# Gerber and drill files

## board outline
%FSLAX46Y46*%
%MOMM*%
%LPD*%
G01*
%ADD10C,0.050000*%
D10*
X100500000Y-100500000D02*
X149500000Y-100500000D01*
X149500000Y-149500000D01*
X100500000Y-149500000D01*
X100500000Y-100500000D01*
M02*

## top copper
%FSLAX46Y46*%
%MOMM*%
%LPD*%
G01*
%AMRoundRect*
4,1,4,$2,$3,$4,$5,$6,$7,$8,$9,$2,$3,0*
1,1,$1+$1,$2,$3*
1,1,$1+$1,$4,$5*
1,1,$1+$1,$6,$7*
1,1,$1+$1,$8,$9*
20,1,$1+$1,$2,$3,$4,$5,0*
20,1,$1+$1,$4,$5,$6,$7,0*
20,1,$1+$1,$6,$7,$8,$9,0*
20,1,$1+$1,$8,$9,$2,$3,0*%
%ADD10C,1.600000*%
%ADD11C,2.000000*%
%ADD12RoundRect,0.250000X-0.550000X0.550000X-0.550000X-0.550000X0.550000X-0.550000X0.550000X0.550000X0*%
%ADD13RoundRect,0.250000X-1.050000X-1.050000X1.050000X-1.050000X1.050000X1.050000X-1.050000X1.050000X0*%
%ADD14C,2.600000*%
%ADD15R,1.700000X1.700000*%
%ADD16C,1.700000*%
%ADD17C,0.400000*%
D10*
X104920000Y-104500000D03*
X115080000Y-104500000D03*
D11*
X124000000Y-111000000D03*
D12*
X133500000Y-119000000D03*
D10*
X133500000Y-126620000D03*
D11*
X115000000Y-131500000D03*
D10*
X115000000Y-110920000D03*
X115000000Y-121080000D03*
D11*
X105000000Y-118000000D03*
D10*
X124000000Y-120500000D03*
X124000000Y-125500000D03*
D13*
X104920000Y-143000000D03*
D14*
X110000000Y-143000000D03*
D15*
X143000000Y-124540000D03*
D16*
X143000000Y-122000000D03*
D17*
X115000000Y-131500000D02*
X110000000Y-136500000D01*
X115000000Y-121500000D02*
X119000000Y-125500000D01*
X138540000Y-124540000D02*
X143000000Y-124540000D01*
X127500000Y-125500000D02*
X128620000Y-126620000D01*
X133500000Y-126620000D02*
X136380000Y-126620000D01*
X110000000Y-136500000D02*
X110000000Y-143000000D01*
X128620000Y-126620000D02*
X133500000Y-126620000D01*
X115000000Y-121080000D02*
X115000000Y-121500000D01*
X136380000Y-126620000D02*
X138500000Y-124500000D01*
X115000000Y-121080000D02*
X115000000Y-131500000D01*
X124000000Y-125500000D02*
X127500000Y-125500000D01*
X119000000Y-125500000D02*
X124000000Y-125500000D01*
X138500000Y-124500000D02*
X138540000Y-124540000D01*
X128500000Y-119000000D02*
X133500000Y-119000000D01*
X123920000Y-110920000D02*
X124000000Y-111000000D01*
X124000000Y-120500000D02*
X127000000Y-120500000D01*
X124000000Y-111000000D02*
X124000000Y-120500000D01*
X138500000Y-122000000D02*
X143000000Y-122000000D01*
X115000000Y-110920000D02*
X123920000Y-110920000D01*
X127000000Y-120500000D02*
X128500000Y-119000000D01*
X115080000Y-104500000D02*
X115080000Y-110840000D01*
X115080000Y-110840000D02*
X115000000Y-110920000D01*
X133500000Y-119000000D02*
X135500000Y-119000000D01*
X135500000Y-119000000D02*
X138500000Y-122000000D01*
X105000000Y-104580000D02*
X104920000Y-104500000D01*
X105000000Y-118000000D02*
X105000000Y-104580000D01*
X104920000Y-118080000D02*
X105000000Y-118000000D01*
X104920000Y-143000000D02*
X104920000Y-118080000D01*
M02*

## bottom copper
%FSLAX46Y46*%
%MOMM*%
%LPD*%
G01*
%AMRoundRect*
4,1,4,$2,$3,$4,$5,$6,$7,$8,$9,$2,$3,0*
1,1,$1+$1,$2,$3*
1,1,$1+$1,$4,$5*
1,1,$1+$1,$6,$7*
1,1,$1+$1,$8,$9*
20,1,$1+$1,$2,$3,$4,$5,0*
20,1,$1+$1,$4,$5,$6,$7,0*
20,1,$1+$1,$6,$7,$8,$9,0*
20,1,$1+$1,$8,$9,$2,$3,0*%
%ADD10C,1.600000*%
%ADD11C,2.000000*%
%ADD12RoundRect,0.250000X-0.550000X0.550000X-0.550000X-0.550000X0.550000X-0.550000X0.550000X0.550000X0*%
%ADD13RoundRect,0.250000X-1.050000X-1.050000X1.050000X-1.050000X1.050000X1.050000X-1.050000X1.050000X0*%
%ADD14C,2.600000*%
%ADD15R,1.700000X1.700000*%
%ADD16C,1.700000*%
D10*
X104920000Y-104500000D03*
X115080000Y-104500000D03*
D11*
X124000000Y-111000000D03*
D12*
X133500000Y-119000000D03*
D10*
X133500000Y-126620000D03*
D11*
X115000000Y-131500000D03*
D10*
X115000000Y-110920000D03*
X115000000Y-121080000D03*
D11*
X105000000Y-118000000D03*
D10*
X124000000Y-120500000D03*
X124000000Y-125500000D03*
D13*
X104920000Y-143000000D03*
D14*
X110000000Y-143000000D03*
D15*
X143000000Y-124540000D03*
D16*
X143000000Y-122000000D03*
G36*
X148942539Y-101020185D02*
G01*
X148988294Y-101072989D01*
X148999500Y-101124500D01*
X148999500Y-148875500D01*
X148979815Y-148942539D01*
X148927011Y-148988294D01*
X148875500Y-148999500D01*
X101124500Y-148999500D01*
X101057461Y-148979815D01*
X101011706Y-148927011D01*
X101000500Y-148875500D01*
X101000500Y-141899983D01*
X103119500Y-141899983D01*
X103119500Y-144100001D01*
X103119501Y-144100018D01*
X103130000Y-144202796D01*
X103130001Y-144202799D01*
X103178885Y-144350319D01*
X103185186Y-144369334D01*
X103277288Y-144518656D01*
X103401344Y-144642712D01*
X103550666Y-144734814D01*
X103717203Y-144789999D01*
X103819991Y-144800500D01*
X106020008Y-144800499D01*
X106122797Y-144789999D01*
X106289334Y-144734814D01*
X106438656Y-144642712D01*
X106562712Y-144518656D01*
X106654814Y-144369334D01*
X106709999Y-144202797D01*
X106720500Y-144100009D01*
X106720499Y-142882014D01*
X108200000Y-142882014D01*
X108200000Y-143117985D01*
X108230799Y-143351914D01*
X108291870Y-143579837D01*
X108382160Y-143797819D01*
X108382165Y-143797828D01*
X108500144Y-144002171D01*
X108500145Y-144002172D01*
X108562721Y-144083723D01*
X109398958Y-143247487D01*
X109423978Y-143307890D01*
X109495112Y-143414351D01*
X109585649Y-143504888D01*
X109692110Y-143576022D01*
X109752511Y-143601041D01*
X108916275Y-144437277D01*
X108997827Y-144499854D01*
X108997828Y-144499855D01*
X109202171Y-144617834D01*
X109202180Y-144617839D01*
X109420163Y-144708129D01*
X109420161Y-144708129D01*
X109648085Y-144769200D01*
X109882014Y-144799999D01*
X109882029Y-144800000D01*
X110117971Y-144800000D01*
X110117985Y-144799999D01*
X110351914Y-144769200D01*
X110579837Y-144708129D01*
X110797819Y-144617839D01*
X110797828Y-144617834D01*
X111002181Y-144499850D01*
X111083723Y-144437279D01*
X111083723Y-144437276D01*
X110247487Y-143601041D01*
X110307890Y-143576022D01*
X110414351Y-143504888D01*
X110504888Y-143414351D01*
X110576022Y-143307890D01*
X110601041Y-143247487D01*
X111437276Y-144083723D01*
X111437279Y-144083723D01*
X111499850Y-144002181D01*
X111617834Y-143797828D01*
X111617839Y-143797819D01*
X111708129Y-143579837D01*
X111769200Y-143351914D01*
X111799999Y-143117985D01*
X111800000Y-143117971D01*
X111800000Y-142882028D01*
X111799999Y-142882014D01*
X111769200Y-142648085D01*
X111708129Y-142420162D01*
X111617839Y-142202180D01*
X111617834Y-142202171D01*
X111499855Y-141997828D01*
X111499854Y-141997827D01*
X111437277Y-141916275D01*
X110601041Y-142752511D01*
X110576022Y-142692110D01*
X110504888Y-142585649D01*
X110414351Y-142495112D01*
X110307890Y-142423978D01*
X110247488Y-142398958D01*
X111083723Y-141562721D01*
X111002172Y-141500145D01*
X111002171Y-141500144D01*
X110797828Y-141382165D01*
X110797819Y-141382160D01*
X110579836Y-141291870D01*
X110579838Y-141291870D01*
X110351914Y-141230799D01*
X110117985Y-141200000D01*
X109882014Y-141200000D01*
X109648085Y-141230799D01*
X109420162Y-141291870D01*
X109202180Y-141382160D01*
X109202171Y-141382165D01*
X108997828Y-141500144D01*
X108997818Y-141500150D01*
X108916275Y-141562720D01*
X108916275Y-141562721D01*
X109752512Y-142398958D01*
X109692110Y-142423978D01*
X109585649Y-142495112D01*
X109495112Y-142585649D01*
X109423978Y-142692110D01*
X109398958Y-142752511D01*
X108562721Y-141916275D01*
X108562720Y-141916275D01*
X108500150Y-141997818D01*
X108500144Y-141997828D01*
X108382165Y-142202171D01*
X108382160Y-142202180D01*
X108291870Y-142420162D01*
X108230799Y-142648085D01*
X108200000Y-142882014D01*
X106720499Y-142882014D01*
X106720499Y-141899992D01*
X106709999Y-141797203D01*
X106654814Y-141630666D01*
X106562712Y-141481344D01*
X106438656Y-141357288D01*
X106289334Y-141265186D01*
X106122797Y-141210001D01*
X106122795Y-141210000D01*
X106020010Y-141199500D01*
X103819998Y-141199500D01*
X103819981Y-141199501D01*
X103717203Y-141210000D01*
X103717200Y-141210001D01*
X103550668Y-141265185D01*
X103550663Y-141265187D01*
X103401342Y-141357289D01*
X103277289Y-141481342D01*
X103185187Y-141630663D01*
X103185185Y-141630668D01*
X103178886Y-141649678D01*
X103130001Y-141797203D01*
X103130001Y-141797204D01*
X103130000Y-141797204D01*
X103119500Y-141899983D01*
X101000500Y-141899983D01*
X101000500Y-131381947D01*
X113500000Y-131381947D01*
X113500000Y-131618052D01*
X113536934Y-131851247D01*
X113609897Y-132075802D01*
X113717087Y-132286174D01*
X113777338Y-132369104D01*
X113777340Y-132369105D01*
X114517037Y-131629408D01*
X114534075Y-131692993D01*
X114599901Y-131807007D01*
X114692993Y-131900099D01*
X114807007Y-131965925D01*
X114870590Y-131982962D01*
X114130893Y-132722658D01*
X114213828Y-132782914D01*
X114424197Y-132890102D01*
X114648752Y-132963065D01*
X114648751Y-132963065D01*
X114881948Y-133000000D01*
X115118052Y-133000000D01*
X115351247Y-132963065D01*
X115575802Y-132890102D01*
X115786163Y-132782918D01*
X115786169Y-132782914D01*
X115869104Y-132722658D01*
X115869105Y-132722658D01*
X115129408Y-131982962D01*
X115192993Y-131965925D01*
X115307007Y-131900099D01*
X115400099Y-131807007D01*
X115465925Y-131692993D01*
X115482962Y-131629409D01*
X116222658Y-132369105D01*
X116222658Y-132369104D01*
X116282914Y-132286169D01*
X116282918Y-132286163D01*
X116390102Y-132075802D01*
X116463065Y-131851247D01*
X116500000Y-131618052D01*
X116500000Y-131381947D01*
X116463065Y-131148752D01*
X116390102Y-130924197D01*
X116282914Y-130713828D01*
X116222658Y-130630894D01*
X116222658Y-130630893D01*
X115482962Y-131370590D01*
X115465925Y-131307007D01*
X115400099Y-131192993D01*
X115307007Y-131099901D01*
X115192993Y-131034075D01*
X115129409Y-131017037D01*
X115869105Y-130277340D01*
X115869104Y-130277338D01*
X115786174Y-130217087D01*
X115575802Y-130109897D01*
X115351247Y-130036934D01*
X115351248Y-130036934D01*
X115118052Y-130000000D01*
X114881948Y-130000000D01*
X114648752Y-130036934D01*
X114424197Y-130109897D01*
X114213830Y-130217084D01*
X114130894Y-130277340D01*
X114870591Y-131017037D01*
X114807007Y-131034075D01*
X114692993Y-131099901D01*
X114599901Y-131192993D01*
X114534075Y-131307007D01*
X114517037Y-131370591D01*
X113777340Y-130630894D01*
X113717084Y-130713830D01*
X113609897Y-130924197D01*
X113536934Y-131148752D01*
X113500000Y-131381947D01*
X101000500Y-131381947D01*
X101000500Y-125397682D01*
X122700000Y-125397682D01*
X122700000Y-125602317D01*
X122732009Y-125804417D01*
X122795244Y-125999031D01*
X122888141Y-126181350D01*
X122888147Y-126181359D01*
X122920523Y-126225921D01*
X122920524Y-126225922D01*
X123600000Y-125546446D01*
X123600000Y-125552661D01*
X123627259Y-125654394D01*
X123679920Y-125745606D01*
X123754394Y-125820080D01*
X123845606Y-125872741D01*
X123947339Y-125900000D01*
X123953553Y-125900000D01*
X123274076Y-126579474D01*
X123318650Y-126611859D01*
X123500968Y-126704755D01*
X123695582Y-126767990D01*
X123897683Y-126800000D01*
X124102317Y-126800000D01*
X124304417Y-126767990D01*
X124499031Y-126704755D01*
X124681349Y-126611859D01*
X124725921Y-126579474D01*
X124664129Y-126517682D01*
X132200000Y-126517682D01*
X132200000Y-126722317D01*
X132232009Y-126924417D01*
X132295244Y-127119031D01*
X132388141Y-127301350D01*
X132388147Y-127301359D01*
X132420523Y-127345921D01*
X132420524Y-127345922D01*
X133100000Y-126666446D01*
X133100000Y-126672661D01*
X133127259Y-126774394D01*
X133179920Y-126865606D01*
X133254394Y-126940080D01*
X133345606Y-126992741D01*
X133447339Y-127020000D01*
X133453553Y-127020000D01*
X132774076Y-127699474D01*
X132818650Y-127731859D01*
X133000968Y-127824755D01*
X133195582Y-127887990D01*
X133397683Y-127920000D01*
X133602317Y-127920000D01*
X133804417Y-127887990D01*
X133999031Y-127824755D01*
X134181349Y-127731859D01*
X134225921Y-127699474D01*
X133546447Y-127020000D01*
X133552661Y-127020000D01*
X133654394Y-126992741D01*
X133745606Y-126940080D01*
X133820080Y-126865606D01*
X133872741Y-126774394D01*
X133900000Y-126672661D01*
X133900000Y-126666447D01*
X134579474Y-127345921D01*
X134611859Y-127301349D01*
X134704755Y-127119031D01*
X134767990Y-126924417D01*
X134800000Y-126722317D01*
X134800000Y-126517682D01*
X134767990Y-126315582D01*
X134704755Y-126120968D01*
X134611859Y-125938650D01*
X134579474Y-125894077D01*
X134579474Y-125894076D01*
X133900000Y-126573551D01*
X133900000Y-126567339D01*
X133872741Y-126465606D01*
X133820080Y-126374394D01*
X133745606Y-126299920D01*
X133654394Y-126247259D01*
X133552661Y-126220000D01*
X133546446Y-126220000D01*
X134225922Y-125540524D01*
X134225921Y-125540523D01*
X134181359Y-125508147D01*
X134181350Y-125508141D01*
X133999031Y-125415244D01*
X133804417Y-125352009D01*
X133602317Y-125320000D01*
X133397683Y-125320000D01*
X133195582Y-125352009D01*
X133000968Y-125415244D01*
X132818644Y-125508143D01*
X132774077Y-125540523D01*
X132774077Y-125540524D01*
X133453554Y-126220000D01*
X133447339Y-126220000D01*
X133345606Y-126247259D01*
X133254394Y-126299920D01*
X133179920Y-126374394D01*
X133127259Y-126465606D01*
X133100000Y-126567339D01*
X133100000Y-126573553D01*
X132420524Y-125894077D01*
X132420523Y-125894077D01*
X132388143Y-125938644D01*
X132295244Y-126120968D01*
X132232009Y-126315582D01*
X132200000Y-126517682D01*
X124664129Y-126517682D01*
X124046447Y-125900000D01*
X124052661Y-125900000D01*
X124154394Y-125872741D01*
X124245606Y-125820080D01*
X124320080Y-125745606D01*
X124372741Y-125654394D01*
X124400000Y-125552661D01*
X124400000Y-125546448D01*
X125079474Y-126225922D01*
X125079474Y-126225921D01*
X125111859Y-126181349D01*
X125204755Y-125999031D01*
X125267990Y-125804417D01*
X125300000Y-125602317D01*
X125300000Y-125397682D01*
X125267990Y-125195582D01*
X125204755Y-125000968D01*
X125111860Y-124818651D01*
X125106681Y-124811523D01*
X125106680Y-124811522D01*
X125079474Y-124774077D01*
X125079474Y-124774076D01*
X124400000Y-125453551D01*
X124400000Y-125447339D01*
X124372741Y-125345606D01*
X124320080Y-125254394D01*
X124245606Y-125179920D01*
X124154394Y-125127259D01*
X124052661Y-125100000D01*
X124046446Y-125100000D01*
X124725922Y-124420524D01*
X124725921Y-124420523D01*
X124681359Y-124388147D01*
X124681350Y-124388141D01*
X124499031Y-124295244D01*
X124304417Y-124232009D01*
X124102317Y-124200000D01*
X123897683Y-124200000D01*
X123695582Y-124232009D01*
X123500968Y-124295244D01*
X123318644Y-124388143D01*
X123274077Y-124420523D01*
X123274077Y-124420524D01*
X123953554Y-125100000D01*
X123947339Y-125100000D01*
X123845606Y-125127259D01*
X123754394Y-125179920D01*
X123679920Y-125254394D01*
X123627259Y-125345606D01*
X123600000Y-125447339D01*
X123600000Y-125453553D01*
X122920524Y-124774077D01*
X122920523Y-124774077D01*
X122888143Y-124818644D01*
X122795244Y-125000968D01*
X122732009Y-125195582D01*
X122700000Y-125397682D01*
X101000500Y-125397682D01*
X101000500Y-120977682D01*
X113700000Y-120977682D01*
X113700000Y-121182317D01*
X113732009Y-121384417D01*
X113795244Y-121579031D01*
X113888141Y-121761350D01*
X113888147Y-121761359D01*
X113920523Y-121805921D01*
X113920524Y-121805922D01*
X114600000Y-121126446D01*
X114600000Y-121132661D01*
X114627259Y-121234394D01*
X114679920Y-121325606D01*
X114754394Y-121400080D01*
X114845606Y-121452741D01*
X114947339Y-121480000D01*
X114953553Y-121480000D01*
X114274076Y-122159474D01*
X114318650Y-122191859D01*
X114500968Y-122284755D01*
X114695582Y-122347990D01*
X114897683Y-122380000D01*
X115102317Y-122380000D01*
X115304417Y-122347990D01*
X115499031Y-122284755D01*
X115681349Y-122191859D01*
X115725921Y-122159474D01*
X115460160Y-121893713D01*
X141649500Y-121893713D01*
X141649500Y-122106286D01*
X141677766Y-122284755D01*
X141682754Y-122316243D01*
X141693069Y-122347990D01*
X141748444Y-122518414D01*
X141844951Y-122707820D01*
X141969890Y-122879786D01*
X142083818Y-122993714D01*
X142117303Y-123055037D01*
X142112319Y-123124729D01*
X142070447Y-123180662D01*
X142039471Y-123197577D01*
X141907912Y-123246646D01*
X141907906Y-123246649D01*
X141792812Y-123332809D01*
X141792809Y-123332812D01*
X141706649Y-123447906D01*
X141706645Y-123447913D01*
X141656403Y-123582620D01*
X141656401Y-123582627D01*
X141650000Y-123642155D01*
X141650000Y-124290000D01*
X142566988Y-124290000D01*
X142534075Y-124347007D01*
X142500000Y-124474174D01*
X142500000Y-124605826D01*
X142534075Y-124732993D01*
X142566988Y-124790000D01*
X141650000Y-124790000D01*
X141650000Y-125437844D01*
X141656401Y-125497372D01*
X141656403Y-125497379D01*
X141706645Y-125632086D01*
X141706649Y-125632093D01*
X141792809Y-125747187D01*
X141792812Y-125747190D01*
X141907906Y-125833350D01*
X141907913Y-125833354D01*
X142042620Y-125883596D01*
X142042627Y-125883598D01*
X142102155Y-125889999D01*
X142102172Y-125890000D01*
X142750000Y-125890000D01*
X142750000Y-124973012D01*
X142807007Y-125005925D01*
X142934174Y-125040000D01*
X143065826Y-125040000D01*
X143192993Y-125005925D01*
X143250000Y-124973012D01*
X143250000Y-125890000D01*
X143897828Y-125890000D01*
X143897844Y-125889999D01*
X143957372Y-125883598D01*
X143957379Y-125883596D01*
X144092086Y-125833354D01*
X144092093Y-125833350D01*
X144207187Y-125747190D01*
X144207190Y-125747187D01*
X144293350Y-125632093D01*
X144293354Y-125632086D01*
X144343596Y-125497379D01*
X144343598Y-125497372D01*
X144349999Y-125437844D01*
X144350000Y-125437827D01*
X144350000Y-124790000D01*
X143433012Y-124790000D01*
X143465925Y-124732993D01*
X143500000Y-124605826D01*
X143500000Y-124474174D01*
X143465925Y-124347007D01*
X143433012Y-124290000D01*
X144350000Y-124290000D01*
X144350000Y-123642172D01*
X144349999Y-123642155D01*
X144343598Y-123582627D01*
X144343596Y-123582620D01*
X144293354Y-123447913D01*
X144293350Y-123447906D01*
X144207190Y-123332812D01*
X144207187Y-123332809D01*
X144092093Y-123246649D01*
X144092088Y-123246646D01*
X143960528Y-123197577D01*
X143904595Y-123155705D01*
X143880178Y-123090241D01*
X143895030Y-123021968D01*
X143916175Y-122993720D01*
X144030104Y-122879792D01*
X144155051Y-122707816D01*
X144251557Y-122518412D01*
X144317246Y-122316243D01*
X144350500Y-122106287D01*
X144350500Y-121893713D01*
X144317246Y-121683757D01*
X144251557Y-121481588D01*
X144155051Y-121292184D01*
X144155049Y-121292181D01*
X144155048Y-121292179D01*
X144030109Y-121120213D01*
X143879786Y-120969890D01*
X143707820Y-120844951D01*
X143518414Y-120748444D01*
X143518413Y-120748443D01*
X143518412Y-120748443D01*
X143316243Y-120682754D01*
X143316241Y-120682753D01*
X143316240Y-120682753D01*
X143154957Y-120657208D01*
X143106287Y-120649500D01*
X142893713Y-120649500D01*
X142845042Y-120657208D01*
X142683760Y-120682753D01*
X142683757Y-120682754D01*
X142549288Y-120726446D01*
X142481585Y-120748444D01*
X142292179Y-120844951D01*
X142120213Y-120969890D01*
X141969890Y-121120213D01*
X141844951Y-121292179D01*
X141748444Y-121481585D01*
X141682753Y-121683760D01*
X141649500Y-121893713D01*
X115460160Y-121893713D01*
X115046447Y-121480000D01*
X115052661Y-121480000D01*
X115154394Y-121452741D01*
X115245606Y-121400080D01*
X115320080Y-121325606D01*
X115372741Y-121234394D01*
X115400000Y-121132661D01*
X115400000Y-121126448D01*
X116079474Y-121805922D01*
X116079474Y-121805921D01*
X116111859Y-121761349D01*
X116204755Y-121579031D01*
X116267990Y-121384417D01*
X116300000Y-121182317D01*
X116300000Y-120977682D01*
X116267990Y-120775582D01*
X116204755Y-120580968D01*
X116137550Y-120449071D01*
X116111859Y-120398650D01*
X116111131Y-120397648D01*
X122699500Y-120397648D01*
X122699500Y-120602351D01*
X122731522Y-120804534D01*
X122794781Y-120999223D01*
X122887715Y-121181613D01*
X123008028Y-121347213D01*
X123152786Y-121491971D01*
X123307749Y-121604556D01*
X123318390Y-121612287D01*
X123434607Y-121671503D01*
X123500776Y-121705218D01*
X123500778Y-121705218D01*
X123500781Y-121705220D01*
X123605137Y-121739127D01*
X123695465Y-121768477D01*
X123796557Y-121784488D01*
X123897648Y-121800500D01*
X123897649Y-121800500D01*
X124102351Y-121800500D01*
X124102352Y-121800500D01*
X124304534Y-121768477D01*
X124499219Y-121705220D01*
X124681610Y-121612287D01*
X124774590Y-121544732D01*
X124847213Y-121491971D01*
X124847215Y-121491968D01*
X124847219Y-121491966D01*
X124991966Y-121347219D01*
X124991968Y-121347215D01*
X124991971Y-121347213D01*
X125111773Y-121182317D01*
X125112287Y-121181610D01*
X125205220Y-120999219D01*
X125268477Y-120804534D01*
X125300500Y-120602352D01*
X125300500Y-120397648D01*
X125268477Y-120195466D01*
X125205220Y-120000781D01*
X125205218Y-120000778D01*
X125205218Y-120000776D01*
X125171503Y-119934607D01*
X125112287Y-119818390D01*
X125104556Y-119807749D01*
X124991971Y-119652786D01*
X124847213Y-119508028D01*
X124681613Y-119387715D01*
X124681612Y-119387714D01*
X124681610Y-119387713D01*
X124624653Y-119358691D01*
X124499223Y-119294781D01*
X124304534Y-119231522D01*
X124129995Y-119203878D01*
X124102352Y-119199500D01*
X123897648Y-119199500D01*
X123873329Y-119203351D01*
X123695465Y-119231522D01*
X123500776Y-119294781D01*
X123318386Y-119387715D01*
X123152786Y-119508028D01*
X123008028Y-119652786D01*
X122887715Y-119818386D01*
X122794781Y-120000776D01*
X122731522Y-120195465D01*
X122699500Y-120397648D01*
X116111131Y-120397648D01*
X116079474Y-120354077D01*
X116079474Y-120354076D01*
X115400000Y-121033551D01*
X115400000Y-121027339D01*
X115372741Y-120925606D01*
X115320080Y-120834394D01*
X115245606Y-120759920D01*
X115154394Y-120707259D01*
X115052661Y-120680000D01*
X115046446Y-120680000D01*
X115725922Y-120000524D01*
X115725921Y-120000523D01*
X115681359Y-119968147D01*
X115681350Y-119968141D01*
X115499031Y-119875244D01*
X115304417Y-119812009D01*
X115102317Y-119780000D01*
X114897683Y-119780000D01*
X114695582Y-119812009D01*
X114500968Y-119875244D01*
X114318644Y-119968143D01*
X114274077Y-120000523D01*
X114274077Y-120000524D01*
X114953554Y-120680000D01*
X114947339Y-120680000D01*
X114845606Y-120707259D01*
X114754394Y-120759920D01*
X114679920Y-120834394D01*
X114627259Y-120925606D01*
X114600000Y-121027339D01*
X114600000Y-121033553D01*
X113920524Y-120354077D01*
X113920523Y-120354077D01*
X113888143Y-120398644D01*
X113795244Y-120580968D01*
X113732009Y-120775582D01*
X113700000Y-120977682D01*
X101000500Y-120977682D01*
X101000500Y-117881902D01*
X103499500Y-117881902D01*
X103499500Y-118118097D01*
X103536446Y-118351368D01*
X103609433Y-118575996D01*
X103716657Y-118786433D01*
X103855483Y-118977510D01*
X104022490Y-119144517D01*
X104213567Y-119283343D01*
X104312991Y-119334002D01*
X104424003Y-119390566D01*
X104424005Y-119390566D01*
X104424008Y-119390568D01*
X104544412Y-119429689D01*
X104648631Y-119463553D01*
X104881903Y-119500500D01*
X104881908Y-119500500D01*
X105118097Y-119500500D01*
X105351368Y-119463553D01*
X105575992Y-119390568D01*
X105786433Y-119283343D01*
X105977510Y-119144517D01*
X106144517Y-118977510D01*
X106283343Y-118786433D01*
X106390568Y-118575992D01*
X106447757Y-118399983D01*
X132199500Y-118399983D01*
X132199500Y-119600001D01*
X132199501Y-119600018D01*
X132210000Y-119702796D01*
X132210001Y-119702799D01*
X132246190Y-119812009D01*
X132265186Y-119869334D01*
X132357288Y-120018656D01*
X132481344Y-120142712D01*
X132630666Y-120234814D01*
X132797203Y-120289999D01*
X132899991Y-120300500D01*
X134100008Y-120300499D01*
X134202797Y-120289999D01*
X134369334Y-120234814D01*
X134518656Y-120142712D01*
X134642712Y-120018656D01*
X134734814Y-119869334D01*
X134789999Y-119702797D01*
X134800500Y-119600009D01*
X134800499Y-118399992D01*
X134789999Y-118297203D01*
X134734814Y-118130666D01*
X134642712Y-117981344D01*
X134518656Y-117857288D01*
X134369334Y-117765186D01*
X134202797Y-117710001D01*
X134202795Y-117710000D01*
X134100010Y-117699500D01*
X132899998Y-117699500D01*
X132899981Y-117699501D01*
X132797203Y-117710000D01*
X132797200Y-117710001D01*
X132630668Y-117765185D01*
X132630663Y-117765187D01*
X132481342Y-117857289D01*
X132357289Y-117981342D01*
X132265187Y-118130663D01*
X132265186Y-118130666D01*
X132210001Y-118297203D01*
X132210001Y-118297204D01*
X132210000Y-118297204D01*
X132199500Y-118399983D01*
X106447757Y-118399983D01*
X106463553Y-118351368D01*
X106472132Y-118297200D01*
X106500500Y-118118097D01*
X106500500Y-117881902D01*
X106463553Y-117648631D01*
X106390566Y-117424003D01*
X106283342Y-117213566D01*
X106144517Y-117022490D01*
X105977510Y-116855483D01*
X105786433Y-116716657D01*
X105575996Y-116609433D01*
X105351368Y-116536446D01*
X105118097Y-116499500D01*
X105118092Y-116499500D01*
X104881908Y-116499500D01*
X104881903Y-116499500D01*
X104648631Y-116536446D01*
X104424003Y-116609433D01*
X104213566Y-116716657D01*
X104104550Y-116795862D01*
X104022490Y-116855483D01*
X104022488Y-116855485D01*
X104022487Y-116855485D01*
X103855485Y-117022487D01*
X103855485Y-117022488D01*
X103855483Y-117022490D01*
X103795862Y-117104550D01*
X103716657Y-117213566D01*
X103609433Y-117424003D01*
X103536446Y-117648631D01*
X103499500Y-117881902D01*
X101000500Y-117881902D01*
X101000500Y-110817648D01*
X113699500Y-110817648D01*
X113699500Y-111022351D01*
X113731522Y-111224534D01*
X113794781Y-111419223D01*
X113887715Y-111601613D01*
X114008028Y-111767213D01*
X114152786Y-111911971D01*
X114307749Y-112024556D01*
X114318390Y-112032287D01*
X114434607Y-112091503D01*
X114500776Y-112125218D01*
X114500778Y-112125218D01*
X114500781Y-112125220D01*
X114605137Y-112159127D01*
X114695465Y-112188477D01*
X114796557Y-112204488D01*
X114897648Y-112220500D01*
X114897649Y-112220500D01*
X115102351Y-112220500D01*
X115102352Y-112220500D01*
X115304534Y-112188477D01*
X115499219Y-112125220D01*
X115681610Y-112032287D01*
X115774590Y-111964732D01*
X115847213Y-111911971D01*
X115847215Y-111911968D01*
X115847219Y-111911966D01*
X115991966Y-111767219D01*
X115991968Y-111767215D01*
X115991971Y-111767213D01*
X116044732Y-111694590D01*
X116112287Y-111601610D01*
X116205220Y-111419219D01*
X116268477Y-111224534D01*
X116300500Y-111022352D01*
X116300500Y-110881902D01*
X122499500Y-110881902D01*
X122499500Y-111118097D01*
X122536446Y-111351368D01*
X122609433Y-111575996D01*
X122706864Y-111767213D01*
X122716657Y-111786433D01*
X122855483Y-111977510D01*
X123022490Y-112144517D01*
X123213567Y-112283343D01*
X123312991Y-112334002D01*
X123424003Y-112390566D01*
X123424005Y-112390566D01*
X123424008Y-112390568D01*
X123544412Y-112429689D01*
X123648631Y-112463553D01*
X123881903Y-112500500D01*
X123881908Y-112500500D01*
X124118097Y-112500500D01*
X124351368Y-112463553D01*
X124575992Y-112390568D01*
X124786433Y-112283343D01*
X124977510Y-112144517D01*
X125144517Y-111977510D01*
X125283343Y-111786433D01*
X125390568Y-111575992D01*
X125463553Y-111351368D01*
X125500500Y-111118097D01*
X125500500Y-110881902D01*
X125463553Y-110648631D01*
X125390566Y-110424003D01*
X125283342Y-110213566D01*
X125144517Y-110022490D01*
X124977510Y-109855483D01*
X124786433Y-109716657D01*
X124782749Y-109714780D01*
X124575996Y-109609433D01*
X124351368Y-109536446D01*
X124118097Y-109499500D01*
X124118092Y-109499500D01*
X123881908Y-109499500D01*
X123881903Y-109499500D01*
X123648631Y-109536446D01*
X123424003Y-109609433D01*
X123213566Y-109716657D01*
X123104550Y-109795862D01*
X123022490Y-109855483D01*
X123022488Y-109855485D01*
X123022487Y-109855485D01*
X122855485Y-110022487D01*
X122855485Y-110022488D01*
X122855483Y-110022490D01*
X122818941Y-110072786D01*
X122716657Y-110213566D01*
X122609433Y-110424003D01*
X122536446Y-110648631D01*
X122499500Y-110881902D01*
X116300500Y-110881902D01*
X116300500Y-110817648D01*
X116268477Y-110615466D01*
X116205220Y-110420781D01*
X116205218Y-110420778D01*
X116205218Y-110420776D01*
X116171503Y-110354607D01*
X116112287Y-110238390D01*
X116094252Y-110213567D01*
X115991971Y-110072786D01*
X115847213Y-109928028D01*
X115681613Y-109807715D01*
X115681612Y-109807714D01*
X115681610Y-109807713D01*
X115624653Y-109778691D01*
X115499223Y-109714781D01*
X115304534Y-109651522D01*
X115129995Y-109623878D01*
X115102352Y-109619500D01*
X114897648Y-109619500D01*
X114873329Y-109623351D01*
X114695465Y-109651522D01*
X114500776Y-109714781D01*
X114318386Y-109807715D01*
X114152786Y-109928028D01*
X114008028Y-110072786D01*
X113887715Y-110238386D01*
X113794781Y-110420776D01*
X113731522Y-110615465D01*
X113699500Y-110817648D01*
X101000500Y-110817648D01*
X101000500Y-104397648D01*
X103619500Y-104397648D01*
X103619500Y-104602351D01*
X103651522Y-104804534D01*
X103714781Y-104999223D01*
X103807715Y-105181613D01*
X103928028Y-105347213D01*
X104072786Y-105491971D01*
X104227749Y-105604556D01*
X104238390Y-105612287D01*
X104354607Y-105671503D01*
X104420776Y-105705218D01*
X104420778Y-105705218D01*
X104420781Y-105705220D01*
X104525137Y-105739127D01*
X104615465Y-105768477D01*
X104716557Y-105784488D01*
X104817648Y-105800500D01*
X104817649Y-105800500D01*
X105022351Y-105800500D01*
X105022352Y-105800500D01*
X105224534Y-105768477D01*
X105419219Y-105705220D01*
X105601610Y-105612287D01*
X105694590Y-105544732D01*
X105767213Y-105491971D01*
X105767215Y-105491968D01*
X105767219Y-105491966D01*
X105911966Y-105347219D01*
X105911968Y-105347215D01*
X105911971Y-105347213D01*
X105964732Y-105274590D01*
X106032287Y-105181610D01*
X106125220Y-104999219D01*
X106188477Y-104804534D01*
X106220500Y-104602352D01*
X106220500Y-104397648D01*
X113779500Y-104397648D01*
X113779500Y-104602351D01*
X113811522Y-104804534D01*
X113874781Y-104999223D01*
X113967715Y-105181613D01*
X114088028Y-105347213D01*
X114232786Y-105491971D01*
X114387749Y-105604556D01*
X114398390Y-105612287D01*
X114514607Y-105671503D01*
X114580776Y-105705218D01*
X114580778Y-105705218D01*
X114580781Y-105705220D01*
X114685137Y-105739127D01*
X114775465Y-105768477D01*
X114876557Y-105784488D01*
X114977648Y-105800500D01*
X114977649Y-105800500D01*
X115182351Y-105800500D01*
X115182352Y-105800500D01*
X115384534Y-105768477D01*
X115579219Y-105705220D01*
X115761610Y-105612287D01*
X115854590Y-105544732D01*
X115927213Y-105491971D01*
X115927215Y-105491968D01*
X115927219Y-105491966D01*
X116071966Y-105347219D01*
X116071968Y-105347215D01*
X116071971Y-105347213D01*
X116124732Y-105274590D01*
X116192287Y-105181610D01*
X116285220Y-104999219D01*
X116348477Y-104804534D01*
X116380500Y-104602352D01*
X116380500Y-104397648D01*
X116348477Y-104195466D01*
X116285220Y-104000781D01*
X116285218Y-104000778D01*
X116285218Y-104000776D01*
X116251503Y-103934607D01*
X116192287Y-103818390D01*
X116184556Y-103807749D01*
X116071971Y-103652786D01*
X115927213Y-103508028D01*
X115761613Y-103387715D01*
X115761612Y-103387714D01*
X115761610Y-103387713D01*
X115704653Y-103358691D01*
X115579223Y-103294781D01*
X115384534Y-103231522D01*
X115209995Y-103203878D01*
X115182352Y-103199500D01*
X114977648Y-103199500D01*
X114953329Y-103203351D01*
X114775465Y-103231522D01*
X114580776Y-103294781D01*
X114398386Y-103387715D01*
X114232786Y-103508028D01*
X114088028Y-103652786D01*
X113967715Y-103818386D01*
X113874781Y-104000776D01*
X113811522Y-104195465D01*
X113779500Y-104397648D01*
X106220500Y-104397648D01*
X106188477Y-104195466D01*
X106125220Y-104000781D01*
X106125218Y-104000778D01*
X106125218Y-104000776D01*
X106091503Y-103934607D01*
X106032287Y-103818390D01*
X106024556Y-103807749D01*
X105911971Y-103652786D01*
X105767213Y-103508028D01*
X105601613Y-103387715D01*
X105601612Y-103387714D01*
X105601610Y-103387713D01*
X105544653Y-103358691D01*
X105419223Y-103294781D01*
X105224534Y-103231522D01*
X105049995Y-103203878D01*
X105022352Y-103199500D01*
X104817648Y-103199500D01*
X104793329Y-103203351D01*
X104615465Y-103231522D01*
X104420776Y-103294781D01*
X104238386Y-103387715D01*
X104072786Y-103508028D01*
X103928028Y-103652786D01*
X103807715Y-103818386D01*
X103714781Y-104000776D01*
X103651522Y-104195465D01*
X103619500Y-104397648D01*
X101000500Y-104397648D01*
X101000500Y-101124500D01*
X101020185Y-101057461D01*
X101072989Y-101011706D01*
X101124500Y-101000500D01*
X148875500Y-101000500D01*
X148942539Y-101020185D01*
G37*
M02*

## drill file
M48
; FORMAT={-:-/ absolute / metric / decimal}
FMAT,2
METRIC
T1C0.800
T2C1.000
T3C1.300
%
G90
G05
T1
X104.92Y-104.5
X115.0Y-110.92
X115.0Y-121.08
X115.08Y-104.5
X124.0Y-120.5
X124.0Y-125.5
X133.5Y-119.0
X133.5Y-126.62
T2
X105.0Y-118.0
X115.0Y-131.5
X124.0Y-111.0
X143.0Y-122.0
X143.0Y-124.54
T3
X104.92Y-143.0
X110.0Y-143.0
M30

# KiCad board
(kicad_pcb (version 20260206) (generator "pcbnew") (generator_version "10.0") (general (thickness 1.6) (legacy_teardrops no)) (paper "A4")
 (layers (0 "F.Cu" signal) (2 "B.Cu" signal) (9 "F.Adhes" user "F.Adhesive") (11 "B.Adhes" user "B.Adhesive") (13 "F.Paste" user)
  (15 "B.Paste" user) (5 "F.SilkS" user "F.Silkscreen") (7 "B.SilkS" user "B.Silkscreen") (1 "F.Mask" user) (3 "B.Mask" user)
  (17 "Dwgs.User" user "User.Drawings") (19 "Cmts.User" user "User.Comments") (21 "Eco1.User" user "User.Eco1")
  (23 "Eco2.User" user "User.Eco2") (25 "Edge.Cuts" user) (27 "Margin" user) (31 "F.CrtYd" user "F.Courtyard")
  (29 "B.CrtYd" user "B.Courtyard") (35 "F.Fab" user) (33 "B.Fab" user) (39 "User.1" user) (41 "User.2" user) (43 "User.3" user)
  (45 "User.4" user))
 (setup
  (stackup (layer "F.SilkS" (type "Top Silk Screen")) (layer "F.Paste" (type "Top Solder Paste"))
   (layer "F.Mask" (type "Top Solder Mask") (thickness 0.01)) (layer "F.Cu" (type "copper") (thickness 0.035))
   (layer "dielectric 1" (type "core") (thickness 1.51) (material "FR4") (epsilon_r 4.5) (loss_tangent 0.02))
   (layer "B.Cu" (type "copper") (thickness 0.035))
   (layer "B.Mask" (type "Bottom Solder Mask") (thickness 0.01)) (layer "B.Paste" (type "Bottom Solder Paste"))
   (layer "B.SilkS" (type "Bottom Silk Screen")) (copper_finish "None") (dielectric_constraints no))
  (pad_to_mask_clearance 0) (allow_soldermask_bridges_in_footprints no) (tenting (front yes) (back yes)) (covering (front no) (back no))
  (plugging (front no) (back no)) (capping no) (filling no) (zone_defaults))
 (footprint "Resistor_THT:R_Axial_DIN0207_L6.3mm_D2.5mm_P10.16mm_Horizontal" (layer "F.Cu") (at 104.92 104.5)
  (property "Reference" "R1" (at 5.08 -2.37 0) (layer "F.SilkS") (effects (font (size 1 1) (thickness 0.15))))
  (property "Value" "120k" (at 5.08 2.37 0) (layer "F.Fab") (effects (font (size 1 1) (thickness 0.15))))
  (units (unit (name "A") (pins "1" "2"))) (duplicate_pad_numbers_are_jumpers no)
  (pad "1" thru_hole circle (at 0 0) (size 1.6 1.6) (drill 0.8) (layers "*.Cu" "*.Mask") (remove_unused_layers no) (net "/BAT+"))
  (pad "2" thru_hole circle (at 10.16 0) (size 1.6 1.6) (drill 0.8) (layers "*.Cu" "*.Mask") (remove_unused_layers no) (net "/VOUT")))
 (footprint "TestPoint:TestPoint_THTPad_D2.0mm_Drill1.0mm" (layer "F.Cu") (at 124 111)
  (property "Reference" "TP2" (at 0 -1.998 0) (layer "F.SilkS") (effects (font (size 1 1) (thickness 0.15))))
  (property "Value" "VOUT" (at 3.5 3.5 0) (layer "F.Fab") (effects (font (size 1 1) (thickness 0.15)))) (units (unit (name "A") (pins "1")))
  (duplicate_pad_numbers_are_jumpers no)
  (pad "1" thru_hole circle (at 0 0) (size 2 2) (drill 1) (layers "*.Cu" "*.Mask") (remove_unused_layers no) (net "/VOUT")))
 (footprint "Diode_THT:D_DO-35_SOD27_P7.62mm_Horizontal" (layer "F.Cu") (at 133.5 119 -90)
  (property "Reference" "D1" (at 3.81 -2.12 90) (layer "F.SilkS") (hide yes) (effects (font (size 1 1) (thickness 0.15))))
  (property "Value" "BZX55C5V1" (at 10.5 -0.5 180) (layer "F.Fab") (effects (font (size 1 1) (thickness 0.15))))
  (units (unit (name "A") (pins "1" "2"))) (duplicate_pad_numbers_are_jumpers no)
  (pad "1" thru_hole roundrect (at 0 0 270) (size 1.6 1.6) (drill 0.8) (layers "*.Cu" "*.Mask") (remove_unused_layers no)
   (roundrect_rratio 0.15625) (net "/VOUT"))
  (pad "2" thru_hole circle (at 7.62 0 270) (size 1.6 1.6) (drill 0.8) (layers "*.Cu" "*.Mask") (remove_unused_layers no) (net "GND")))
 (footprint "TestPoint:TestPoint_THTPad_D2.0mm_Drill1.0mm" (layer "F.Cu") (at 115 131.5)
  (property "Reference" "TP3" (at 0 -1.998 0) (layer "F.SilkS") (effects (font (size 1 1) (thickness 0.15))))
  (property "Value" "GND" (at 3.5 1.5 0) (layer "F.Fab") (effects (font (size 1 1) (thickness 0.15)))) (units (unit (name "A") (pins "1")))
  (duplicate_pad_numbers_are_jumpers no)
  (pad "1" thru_hole circle (at 0 0) (size 2 2) (drill 1) (layers "*.Cu" "*.Mask") (remove_unused_layers no) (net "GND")))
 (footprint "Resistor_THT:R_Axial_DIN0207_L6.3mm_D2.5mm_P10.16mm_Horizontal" (layer "F.Cu") (at 115 110.92 -90)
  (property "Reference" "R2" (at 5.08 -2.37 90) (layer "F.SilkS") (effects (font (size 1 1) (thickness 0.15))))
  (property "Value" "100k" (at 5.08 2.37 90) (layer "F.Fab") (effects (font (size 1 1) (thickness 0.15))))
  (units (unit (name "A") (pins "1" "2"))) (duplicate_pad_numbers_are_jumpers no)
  (pad "1" thru_hole circle (at 0 0 270) (size 1.6 1.6) (drill 0.8) (layers "*.Cu" "*.Mask") (remove_unused_layers no) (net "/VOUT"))
  (pad "2" thru_hole circle (at 10.16 0 270) (size 1.6 1.6) (drill 0.8) (layers "*.Cu" "*.Mask") (remove_unused_layers no) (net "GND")))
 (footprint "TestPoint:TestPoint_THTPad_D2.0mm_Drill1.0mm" (layer "F.Cu") (at 105 118)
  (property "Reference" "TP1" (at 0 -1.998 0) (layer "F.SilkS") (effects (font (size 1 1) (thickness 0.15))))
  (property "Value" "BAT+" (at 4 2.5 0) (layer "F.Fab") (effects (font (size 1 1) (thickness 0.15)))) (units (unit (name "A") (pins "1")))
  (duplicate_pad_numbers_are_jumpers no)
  (pad "1" thru_hole circle (at 0 0) (size 2 2) (drill 1) (layers "*.Cu" "*.Mask") (remove_unused_layers no) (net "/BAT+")))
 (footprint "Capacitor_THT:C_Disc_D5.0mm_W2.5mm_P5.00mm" (layer "F.Cu") (at 124 120.5 -90)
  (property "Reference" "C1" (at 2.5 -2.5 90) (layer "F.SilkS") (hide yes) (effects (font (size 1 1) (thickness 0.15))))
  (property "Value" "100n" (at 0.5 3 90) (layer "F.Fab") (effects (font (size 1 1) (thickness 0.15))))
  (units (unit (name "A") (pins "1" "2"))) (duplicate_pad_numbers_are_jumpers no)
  (pad "1" thru_hole circle (at 0 0 270) (size 1.6 1.6) (drill 0.8) (layers "*.Cu" "*.Mask") (remove_unused_layers no) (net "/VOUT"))
  (pad "2" thru_hole circle (at 5 0 270) (size 1.6 1.6) (drill 0.8) (layers "*.Cu" "*.Mask") (remove_unused_layers no) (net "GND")))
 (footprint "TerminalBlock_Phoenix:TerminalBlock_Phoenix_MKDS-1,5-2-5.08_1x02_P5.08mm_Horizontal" (layer "F.Cu") (at 104.92 143)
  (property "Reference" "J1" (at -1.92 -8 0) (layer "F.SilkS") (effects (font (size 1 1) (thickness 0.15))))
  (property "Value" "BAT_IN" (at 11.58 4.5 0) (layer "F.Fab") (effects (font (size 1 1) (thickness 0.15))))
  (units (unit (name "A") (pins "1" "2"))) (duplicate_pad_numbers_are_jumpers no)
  (pad "1" thru_hole roundrect (at 0 0) (size 2.6 2.6) (drill 1.3) (layers "*.Cu" "*.Mask") (remove_unused_layers no)
   (roundrect_rratio 0.096154) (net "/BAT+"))
  (pad "2" thru_hole circle (at 5.08 0) (size 2.6 2.6) (drill 1.3) (layers "*.Cu" "*.Mask") (remove_unused_layers no) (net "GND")))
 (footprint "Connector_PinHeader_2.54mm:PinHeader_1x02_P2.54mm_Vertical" (layer "F.Cu") (at 143 124.54 180)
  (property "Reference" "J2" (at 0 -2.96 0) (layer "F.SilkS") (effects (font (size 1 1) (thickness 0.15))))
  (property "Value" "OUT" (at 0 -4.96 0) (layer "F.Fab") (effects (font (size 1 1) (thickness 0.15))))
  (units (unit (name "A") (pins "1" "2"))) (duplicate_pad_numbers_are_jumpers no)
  (pad "1" thru_hole rect (at 0 0 180) (size 1.7 1.7) (drill 1) (layers "*.Cu" "*.Mask") (remove_unused_layers no) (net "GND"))
  (pad "2" thru_hole circle (at 0 2.54 180) (size 1.7 1.7) (drill 1) (layers "*.Cu" "*.Mask") (remove_unused_layers no) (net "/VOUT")))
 (gr_rect (start 100.5 100.5) (end 149.5 149.5) (stroke (width 0.05) (type solid)) (fill no) (layer "Edge.Cuts"))
 (segment (start 115 131.5) (end 110 136.5) (width 0.4) (layer "F.Cu") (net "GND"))
 (segment (start 115 121.5) (end 119 125.5) (width 0.4) (layer "F.Cu") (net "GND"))
 (segment (start 138.54 124.54) (end 143 124.54) (width 0.4) (layer "F.Cu") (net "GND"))
 (segment (start 127.5 125.5) (end 128.62 126.62) (width 0.4) (layer "F.Cu") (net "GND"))
 (segment (start 133.5 126.62) (end 136.38 126.62) (width 0.4) (layer "F.Cu") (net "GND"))
 (segment (start 110 136.5) (end 110 143) (width 0.4) (layer "F.Cu") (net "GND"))
 (segment (start 128.62 126.62) (end 133.5 126.62) (width 0.4) (layer "F.Cu") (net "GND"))
 (segment (start 115 121.08) (end 115 121.5) (width 0.4) (layer "F.Cu") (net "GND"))
 (segment (start 136.38 126.62) (end 138.5 124.5) (width 0.4) (layer "F.Cu") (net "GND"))
 (segment (start 115 121.08) (end 115 131.5) (width 0.4) (layer "F.Cu") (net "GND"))
 (segment (start 124 125.5) (end 127.5 125.5) (width 0.4) (layer "F.Cu") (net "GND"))
 (segment (start 119 125.5) (end 124 125.5) (width 0.4) (layer "F.Cu") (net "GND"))
 (segment (start 138.5 124.5) (end 138.54 124.54) (width 0.4) (layer "F.Cu") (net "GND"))
 (segment (start 128.5 119) (end 133.5 119) (width 0.4) (layer "F.Cu") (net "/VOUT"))
 (segment (start 123.92 110.92) (end 124 111) (width 0.4) (layer "F.Cu") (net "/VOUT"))
 (segment (start 124 120.5) (end 127 120.5) (width 0.4) (layer "F.Cu") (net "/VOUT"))
 (segment (start 124 111) (end 124 120.5) (width 0.4) (layer "F.Cu") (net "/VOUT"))
 (segment (start 138.5 122) (end 143 122) (width 0.4) (layer "F.Cu") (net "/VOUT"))
 (segment (start 115 110.92) (end 123.92 110.92) (width 0.4) (layer "F.Cu") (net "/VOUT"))
 (segment (start 127 120.5) (end 128.5 119) (width 0.4) (layer "F.Cu") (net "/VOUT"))
 (segment (start 115.08 104.5) (end 115.08 110.84) (width 0.4) (layer "F.Cu") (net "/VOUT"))
 (segment (start 115.08 110.84) (end 115 110.92) (width 0.4) (layer "F.Cu") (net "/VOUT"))
 (segment (start 133.5 119) (end 135.5 119) (width 0.4) (layer "F.Cu") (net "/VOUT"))
 (segment (start 135.5 119) (end 138.5 122) (width 0.4) (layer "F.Cu") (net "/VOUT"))
 (segment (start 105 104.58) (end 104.92 104.5) (width 0.4) (layer "F.Cu") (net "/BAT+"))
 (segment (start 105 118) (end 105 104.58) (width 0.4) (layer "F.Cu") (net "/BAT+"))
 (segment (start 104.92 118.08) (end 105 118) (width 0.4) (layer "F.Cu") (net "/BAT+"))
 (segment (start 104.92 143) (end 104.92 118.08) (width 0.4) (layer "F.Cu") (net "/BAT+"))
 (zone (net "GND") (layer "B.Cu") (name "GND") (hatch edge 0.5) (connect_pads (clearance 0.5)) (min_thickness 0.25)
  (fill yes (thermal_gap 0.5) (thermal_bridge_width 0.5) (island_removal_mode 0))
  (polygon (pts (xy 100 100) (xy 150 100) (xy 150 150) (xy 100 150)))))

